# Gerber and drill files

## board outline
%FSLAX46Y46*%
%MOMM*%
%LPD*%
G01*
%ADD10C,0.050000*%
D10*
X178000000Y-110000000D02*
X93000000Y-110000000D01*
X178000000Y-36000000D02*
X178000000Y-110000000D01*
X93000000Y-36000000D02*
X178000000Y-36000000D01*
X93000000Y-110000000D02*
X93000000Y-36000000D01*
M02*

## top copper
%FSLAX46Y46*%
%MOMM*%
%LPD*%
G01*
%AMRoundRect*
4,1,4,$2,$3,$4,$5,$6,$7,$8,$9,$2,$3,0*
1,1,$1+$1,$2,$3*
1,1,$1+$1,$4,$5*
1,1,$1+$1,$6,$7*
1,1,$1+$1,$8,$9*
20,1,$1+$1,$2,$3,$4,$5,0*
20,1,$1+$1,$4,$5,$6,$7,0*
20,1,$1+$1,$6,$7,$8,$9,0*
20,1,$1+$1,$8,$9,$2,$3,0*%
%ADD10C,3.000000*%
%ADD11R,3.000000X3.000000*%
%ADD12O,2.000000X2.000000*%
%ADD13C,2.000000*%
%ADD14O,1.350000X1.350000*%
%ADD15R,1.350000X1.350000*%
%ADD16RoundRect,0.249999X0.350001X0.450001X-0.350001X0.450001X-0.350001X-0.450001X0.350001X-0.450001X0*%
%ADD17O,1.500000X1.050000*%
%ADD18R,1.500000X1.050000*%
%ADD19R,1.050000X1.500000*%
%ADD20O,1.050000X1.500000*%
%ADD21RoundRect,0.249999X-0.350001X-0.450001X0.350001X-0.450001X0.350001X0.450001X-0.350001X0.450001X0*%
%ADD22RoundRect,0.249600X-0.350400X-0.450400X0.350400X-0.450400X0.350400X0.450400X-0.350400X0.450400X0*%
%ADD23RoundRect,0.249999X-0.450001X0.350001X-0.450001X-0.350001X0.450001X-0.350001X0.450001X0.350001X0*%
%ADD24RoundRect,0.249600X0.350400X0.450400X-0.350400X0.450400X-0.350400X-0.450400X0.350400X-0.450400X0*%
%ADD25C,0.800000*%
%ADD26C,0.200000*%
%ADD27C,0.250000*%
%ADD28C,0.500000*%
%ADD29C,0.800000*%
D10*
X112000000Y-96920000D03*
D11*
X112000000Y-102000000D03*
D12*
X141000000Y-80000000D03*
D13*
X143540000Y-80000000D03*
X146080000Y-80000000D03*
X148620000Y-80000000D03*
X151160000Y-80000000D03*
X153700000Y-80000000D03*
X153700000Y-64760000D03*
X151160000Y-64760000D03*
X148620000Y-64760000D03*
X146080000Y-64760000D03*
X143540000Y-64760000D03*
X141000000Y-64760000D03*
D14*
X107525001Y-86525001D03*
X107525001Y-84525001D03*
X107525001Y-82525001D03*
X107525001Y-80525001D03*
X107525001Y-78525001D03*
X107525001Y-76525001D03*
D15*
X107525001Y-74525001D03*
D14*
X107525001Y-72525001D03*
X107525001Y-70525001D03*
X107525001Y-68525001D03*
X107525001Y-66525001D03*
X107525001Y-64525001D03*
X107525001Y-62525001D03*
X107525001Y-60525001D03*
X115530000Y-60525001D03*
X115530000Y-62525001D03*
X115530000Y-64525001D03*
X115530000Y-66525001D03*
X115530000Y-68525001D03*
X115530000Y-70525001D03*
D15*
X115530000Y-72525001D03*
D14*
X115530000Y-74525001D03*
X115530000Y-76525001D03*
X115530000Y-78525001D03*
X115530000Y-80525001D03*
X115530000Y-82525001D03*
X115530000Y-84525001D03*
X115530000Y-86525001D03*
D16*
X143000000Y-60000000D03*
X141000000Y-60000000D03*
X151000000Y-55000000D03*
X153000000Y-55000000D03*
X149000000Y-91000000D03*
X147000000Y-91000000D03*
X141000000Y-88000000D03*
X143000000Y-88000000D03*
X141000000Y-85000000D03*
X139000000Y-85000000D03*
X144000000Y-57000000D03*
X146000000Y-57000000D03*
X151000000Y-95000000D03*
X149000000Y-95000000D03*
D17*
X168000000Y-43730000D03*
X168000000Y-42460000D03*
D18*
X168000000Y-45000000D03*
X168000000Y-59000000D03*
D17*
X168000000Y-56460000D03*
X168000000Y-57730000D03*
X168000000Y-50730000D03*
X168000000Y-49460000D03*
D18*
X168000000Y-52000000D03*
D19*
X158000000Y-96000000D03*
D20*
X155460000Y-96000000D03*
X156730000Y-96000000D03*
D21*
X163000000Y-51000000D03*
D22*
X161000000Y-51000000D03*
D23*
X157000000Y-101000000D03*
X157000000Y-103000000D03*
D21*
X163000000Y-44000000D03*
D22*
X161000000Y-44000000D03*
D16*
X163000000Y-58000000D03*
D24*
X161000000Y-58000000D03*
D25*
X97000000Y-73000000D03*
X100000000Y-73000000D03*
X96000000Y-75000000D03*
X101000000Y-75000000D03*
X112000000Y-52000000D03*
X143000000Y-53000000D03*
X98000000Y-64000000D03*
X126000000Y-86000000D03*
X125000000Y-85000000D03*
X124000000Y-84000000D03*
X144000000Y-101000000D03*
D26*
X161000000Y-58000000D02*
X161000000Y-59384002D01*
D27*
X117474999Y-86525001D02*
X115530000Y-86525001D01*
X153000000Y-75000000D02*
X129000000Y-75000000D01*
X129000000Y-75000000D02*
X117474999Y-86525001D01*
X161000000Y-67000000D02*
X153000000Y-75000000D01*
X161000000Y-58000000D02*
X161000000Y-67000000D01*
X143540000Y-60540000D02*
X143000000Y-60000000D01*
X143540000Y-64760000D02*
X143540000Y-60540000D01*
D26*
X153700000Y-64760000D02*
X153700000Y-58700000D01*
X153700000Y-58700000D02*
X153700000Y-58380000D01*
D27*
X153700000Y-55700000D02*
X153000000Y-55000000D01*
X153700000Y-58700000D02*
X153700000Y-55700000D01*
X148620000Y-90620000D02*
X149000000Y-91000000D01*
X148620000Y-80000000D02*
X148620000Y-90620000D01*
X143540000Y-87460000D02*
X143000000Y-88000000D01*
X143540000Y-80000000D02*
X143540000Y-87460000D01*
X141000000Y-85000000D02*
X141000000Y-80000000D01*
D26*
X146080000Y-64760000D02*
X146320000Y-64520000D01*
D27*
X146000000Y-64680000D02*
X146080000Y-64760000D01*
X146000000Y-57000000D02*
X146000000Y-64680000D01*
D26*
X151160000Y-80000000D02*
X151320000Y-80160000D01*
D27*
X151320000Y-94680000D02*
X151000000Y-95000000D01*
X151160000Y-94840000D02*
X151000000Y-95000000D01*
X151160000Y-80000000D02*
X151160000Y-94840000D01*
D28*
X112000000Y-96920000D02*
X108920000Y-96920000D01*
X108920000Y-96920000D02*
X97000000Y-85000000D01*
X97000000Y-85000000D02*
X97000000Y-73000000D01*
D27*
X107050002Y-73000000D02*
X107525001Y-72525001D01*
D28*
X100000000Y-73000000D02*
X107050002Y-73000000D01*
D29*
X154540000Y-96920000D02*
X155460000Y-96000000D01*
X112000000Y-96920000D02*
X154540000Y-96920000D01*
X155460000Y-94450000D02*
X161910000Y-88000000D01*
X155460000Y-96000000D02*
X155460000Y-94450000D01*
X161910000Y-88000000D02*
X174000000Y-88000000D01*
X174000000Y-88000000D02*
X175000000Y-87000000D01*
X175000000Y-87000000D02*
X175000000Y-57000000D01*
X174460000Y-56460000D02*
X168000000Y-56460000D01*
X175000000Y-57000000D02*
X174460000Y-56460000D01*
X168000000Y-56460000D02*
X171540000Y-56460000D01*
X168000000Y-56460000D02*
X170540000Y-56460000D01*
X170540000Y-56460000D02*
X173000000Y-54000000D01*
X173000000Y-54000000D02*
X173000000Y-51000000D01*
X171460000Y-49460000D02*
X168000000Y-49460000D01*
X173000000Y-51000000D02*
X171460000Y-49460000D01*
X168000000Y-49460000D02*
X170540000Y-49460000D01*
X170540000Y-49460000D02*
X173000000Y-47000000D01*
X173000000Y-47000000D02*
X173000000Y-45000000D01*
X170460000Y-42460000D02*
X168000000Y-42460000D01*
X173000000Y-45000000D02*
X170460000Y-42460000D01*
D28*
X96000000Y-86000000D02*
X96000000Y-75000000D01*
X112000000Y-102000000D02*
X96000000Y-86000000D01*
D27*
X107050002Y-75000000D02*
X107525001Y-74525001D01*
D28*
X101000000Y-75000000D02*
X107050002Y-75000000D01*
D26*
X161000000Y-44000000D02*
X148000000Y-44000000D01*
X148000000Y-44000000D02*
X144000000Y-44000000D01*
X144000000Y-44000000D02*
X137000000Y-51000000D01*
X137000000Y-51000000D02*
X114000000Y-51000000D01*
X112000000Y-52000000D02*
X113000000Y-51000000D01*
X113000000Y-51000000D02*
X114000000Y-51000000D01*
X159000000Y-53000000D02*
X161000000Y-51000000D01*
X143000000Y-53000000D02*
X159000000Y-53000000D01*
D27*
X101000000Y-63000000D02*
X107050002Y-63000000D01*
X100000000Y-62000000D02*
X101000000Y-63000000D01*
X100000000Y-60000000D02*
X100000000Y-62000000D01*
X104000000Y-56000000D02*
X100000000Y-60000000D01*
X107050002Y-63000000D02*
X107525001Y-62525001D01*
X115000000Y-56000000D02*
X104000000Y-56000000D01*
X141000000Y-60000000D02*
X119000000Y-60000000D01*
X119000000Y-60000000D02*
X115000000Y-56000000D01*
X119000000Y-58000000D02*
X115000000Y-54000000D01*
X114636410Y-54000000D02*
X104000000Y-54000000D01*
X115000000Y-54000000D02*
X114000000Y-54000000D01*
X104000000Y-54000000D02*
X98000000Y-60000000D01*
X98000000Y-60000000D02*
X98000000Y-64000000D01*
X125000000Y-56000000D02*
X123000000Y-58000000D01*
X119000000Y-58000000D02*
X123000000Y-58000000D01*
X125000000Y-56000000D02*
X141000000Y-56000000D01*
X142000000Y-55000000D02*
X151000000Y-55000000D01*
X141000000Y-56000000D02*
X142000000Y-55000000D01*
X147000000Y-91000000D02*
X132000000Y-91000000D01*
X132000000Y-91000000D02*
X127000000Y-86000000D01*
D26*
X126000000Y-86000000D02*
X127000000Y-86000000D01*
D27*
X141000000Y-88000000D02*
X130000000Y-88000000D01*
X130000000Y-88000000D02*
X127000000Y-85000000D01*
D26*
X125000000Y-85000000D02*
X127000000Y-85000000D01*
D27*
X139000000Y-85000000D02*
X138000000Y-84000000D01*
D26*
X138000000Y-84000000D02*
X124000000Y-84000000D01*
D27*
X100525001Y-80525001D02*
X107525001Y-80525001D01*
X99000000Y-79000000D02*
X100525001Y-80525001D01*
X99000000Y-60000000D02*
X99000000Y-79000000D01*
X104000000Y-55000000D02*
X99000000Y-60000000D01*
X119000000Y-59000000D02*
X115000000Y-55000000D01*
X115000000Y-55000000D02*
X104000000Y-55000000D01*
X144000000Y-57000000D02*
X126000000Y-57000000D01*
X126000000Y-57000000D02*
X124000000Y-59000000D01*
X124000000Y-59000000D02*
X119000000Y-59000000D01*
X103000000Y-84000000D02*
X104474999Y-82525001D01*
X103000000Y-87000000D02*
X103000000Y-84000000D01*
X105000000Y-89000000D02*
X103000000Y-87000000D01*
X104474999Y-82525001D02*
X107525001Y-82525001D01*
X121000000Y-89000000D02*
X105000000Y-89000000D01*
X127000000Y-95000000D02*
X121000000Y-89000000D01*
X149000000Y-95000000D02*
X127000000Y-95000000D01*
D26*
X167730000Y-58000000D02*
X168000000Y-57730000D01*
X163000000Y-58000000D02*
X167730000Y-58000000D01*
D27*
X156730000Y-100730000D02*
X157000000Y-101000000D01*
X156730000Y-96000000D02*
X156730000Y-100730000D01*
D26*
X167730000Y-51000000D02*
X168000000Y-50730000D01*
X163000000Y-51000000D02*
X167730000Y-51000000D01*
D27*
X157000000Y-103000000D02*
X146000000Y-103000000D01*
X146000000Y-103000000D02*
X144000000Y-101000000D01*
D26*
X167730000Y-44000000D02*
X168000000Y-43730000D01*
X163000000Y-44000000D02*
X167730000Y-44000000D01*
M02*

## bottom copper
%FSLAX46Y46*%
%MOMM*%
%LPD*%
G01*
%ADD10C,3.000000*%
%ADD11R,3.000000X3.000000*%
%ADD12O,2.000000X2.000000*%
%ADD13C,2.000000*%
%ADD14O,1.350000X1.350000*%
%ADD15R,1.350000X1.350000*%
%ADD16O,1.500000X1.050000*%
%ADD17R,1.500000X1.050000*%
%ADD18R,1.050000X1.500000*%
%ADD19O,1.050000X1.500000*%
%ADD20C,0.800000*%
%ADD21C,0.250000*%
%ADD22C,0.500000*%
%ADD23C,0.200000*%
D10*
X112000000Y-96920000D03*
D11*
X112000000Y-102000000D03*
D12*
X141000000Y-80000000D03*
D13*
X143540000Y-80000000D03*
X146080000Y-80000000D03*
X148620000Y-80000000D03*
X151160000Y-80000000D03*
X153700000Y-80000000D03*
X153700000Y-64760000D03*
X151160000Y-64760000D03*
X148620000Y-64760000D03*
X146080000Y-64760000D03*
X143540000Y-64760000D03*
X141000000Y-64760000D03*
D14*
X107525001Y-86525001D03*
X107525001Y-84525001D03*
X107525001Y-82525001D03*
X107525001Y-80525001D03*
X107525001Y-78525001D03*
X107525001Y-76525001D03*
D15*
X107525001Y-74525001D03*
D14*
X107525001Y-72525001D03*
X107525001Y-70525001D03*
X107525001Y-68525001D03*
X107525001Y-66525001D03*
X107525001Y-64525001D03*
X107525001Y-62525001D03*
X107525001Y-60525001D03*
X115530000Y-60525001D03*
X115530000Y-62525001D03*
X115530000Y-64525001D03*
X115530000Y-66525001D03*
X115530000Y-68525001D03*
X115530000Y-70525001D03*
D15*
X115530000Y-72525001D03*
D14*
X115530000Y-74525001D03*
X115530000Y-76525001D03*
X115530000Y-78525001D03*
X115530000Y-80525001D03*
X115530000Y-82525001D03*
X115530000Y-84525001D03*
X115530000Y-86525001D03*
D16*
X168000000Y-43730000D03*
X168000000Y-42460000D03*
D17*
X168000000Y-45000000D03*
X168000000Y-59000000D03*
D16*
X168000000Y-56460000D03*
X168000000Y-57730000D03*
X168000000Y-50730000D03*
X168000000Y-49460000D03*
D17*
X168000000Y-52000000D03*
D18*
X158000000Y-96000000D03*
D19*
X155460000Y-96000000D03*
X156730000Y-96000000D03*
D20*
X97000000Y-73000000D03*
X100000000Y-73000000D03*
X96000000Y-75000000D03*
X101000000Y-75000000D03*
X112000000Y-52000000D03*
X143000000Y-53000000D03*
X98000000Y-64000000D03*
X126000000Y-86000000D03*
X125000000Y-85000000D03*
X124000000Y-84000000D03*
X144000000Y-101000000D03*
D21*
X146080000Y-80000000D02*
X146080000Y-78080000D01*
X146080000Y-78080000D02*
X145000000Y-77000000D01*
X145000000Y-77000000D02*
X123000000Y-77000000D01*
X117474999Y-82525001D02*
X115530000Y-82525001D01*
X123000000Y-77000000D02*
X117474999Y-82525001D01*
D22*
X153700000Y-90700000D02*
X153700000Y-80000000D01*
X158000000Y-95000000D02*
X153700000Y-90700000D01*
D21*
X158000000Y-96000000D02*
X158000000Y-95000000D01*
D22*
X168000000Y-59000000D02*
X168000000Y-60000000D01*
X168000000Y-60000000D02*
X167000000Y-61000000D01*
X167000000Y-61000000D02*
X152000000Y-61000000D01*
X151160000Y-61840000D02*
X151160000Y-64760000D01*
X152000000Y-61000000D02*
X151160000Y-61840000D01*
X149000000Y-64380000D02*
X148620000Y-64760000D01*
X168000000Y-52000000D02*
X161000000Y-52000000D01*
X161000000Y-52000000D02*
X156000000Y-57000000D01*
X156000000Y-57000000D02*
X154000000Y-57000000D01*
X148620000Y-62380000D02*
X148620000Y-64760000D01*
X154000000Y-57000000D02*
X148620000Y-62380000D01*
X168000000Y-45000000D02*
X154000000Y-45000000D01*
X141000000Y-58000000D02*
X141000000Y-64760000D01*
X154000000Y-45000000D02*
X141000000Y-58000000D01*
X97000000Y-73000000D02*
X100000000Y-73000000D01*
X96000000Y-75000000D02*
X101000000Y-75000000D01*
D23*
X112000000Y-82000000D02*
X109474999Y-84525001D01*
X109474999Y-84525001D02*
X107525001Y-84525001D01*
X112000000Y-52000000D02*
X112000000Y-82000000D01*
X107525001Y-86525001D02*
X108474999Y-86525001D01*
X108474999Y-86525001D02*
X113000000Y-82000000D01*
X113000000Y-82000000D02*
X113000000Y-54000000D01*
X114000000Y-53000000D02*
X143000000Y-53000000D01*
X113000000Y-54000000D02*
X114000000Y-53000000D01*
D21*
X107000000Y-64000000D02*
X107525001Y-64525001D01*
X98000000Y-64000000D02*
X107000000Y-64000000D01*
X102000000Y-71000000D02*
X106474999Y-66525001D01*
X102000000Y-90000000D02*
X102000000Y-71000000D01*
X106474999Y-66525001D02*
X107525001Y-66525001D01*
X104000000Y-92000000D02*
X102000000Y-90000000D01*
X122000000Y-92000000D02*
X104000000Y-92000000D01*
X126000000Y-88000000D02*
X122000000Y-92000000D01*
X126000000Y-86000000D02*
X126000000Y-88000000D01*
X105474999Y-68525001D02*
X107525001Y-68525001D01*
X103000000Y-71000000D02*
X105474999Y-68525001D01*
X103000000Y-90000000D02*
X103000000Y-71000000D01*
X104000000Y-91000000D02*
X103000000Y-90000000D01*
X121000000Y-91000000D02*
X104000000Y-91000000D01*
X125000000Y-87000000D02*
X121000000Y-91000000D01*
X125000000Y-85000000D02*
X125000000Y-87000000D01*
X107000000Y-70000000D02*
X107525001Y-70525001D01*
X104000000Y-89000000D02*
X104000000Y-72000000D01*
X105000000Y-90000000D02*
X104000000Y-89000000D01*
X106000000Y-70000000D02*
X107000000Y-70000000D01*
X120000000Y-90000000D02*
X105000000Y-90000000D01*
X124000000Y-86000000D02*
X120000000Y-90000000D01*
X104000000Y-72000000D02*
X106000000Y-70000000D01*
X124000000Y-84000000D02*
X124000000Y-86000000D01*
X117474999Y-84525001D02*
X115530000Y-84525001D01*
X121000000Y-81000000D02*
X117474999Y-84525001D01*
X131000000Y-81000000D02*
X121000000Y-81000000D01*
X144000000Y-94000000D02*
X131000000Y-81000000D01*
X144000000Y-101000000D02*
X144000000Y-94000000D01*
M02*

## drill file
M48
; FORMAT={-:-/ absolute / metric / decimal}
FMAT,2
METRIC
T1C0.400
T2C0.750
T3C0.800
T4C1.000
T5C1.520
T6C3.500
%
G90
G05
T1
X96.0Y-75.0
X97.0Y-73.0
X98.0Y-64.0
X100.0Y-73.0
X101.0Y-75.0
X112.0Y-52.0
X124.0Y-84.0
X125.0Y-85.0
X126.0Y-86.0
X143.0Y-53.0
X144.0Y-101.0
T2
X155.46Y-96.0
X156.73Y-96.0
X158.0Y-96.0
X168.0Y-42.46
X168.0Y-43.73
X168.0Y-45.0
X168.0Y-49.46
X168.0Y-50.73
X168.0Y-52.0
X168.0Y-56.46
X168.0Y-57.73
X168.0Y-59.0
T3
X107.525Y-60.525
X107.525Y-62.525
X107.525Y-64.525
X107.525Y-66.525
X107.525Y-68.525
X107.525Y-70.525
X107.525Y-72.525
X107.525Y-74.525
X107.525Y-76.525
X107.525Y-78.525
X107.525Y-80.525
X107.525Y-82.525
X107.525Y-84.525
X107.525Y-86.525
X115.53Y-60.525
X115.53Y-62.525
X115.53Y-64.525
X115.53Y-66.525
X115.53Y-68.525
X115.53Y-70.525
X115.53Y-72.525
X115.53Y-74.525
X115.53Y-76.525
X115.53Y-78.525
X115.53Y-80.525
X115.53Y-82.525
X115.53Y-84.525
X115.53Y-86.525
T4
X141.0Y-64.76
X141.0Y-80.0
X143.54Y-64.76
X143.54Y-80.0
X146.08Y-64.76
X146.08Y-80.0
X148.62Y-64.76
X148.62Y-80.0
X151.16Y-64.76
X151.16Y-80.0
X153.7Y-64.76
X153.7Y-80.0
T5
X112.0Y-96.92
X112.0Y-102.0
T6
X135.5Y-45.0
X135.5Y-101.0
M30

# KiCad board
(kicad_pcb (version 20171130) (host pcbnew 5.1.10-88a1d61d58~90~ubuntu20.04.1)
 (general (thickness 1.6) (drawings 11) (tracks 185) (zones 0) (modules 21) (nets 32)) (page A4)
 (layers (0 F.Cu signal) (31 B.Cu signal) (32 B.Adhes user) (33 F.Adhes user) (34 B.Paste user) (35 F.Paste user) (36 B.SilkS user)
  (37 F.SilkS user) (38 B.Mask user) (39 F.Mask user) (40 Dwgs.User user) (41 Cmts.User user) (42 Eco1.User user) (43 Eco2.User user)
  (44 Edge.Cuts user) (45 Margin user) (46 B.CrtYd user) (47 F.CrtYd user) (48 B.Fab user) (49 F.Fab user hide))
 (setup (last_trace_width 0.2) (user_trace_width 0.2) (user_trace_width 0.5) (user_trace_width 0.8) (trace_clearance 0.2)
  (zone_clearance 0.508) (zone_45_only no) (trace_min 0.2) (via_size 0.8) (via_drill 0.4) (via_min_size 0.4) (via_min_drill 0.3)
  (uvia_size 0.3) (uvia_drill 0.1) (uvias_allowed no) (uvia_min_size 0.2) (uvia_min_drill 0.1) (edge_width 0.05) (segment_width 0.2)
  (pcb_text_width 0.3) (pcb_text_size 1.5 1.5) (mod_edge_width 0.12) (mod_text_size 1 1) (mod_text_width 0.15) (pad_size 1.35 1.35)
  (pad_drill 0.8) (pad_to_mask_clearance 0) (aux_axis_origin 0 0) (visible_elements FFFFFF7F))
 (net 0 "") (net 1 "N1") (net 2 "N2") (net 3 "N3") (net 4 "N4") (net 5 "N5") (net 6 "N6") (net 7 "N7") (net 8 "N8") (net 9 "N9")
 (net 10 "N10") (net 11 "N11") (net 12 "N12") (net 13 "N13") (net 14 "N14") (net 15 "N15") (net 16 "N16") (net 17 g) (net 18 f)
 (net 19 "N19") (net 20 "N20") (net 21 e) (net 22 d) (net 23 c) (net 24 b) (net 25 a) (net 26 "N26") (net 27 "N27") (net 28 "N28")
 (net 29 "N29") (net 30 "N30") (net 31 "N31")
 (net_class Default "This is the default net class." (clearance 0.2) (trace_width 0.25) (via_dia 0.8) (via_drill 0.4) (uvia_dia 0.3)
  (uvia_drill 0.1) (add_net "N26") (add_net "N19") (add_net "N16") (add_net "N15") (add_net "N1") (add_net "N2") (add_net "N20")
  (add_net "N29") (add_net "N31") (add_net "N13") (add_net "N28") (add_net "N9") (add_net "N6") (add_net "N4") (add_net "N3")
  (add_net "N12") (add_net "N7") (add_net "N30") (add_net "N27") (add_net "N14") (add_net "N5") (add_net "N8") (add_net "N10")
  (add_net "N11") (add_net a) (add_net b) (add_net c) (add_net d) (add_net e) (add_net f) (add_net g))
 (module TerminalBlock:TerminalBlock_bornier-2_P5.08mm (layer F.Cu) (at 112 102 90)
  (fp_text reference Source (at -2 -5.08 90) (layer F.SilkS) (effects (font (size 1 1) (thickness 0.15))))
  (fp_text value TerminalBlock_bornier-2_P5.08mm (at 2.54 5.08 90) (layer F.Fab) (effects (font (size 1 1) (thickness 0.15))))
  (pad 2 thru_hole circle (at 5.08 0 90) (size 3 3) (drill 1.52) (layers *.Cu *.Mask) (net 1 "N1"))
  (pad 1 thru_hole rect (at 0 0 90) (size 3 3) (drill 1.52) (layers *.Cu *.Mask) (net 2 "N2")))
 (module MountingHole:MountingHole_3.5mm (layer F.Cu) (at 135.5 45)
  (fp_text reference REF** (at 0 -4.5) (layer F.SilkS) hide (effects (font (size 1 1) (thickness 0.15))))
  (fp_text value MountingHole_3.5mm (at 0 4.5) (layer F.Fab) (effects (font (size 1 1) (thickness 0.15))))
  (pad 1 np_thru_hole circle (at 0 0) (size 3.5 3.5) (drill 3.5) (layers *.Cu *.Mask)))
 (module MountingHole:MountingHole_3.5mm (layer F.Cu) (at 135.5 101)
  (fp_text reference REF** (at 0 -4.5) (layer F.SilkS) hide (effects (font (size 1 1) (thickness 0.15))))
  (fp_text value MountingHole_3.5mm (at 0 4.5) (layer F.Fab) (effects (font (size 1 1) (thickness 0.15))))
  (pad 1 np_thru_hole circle (at 0 0) (size 3.5 3.5) (drill 3.5) (layers *.Cu *.Mask)))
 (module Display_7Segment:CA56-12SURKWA (layer F.Cu) (at 141 80 90)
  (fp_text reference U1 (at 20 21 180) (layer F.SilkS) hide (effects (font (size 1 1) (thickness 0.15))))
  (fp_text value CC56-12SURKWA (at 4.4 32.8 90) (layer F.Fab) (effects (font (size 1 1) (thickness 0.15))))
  (pad 1 thru_hole oval (at 0 0 90) (size 2 2) (drill 1) (layers *.Cu *.Mask) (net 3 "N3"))
  (pad 2 thru_hole circle (at 0 2.54 90) (size 2 2) (drill 1) (layers *.Cu *.Mask) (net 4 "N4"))
  (pad 3 thru_hole circle (at 0 5.08 90) (size 2 2) (drill 1) (layers *.Cu *.Mask) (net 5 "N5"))
  (pad 4 thru_hole circle (at 0 7.62 90) (size 2 2) (drill 1) (layers *.Cu *.Mask) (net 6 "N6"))
  (pad 5 thru_hole circle (at 0 10.16 90) (size 2 2) (drill 1) (layers *.Cu *.Mask) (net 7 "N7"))
  (pad 6 thru_hole circle (at 0 12.7 90) (size 2 2) (drill 1) (layers *.Cu *.Mask) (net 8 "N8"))
  (pad 7 thru_hole circle (at 15.24 12.7 90) (size 2 2) (drill 1) (layers *.Cu *.Mask) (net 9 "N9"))
  (pad 8 thru_hole circle (at 15.24 10.16 90) (size 2 2) (drill 1) (layers *.Cu *.Mask) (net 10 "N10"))
  (pad 9 thru_hole circle (at 15.24 7.62 90) (size 2 2) (drill 1) (layers *.Cu *.Mask) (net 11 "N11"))
  (pad 10 thru_hole circle (at 15.24 5.08 90) (size 2 2) (drill 1) (layers *.Cu *.Mask) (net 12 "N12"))
  (pad 11 thru_hole circle (at 15.24 2.54 90) (size 2 2) (drill 1) (layers *.Cu *.Mask) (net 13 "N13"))
  (pad 12 thru_hole circle (at 15.24 0 90) (size 2 2) (drill 1) (layers *.Cu *.Mask) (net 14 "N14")))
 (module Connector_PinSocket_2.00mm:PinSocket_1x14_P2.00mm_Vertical (layer F.Cu) (at 107.525001 60.525001)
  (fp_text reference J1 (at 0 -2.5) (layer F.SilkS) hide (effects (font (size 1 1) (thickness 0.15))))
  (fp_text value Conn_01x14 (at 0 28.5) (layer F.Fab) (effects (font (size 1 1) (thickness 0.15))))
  (pad 14 thru_hole oval (at 0 26) (size 1.35 1.35) (drill 0.8) (layers *.Cu *.Mask) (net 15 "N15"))
  (pad 13 thru_hole oval (at 0 24) (size 1.35 1.35) (drill 0.8) (layers *.Cu *.Mask) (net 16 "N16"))
  (pad 12 thru_hole oval (at 0 22) (size 1.35 1.35) (drill 0.8) (layers *.Cu *.Mask) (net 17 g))
  (pad 11 thru_hole oval (at 0 20) (size 1.35 1.35) (drill 0.8) (layers *.Cu *.Mask) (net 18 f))
  (pad 10 thru_hole oval (at 0 18) (size 1.35 1.35) (drill 0.8) (layers *.Cu *.Mask) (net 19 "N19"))
  (pad 9 thru_hole oval (at 0 16) (size 1.35 1.35) (drill 0.8) (layers *.Cu *.Mask) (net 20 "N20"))
  (pad 8 thru_hole rect (at 0 14) (size 1.35 1.35) (drill 0.8) (layers *.Cu *.Mask) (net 2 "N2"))
  (pad 7 thru_hole oval (at 0 12) (size 1.35 1.35) (drill 0.8) (layers *.Cu *.Mask) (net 1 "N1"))
  (pad 6 thru_hole oval (at 0 10) (size 1.35 1.35) (drill 0.8) (layers *.Cu *.Mask) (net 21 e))
  (pad 5 thru_hole oval (at 0 8) (size 1.35 1.35) (drill 0.8) (layers *.Cu *.Mask) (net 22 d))
  (pad 4 thru_hole oval (at 0 6) (size 1.35 1.35) (drill 0.8) (layers *.Cu *.Mask) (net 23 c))
  (pad 3 thru_hole oval (at 0 4) (size 1.35 1.35) (drill 0.8) (layers *.Cu *.Mask) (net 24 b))
  (pad 2 thru_hole oval (at 0 2) (size 1.35 1.35) (drill 0.8) (layers *.Cu *.Mask) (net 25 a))
  (pad 1 thru_hole oval (at 0 0) (size 1.35 1.35) (drill 0.8) (layers *.Cu *.Mask) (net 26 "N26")))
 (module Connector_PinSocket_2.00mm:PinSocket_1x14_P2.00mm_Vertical (layer F.Cu) (at 115.53 60.525001)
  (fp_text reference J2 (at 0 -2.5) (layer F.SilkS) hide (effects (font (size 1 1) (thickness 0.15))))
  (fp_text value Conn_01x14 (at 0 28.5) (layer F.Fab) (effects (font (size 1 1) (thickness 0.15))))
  (pad 28 thru_hole oval (at 0 0) (size 1.35 1.35) (drill 0.8) (layers *.Cu *.Mask))
  (pad 27 thru_hole oval (at 0 2) (size 1.35 1.35) (drill 0.8) (layers *.Cu *.Mask))
  (pad 26 thru_hole oval (at 0 4) (size 1.35 1.35) (drill 0.8) (layers *.Cu *.Mask))
  (pad 25 thru_hole oval (at 0 6) (size 1.35 1.35) (drill 0.8) (layers *.Cu *.Mask))
  (pad 24 thru_hole oval (at 0 8) (size 1.35 1.35) (drill 0.8) (layers *.Cu *.Mask))
  (pad 23 thru_hole oval (at 0 10) (size 1.35 1.35) (drill 0.8) (layers *.Cu *.Mask))
  (pad 22 thru_hole rect (at 0 12) (size 1.35 1.35) (drill 0.8) (layers *.Cu *.Mask))
  (pad 21 thru_hole oval (at 0 14) (size 1.35 1.35) (drill 0.8) (layers *.Cu *.Mask))
  (pad 20 thru_hole oval (at 0 16) (size 1.35 1.35) (drill 0.8) (layers *.Cu *.Mask))
  (pad 19 thru_hole oval (at 0 18) (size 1.35 1.35) (drill 0.8) (layers *.Cu *.Mask))
  (pad 18 thru_hole oval (at 0 20) (size 1.35 1.35) (drill 0.8) (layers *.Cu *.Mask))
  (pad 17 thru_hole oval (at 0 22) (size 1.35 1.35) (drill 0.8) (layers *.Cu *.Mask) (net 5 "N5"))
  (pad 16 thru_hole oval (at 0 24) (size 1.35 1.35) (drill 0.8) (layers *.Cu *.Mask) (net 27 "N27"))
  (pad 15 thru_hole oval (at 0 26) (size 1.35 1.35) (drill 0.8) (layers *.Cu *.Mask)))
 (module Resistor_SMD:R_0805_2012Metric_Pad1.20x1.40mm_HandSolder (layer F.Cu) (at 142 60 180)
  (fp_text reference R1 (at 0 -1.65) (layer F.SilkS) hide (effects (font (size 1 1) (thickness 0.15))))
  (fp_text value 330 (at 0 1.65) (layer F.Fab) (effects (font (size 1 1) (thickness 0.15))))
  (pad 1 smd roundrect (at -1 0 180) (size 1.2 1.4) (layers F.Cu F.Paste F.Mask) (roundrect_rratio 0.2083325) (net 13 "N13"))
  (pad 2 smd roundrect (at 1 0 180) (size 1.2 1.4) (layers F.Cu F.Paste F.Mask) (roundrect_rratio 0.2083325) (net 25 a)))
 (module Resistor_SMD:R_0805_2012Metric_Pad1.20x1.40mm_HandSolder (layer F.Cu) (at 152 55 180)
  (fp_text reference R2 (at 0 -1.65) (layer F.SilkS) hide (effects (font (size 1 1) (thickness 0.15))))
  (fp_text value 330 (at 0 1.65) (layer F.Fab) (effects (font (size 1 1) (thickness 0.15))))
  (pad 2 smd roundrect (at 1 0 180) (size 1.2 1.4) (layers F.Cu F.Paste F.Mask) (roundrect_rratio 0.2083325) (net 24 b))
  (pad 1 smd roundrect (at -1 0 180) (size 1.2 1.4) (layers F.Cu F.Paste F.Mask) (roundrect_rratio 0.2083325) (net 9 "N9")))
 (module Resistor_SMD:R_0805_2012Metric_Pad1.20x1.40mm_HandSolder (layer F.Cu) (at 148 91 180)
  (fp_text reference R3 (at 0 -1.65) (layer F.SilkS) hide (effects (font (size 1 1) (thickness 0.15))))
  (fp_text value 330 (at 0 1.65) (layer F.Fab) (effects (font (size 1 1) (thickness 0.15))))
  (pad 1 smd roundrect (at -1 0 180) (size 1.2 1.4) (layers F.Cu F.Paste F.Mask) (roundrect_rratio 0.2083325) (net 6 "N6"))
  (pad 2 smd roundrect (at 1 0 180) (size 1.2 1.4) (layers F.Cu F.Paste F.Mask) (roundrect_rratio 0.2083325) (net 23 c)))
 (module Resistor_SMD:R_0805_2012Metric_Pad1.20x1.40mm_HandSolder (layer F.Cu) (at 142 88 180)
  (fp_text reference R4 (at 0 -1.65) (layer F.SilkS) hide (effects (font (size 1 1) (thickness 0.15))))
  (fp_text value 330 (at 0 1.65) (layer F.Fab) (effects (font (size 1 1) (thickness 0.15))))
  (pad 2 smd roundrect (at 1 0 180) (size 1.2 1.4) (layers F.Cu F.Paste F.Mask) (roundrect_rratio 0.2083325) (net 22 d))
  (pad 1 smd roundrect (at -1 0 180) (size 1.2 1.4) (layers F.Cu F.Paste F.Mask) (roundrect_rratio 0.2083325) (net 4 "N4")))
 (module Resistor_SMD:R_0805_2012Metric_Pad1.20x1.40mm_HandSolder (layer F.Cu) (at 140 85 180)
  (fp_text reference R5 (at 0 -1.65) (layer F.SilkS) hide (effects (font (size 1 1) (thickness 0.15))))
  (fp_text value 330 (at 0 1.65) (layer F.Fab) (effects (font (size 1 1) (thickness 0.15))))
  (pad 1 smd roundrect (at -1 0 180) (size 1.2 1.4) (layers F.Cu F.Paste F.Mask) (roundrect_rratio 0.2083325) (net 3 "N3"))
  (pad 2 smd roundrect (at 1 0 180) (size 1.2 1.4) (layers F.Cu F.Paste F.Mask) (roundrect_rratio 0.2083325) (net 21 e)))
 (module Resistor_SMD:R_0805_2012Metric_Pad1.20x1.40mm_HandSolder (layer F.Cu) (at 145 57 180)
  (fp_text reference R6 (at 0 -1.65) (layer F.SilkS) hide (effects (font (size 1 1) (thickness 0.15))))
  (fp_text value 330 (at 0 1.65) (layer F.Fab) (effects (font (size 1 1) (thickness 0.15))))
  (pad 2 smd roundrect (at 1 0 180) (size 1.2 1.4) (layers F.Cu F.Paste F.Mask) (roundrect_rratio 0.2083325) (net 18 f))
  (pad 1 smd roundrect (at -1 0 180) (size 1.2 1.4) (layers F.Cu F.Paste F.Mask) (roundrect_rratio 0.2083325) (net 12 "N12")))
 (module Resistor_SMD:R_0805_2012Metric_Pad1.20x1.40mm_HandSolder (layer F.Cu) (at 150 95 180)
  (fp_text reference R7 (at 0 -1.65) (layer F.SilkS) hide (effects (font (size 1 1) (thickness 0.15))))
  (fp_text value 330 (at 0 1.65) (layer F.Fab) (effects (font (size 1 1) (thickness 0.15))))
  (pad 1 smd roundrect (at -1 0 180) (size 1.2 1.4) (layers F.Cu F.Paste F.Mask) (roundrect_rratio 0.2083325) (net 7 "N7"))
  (pad 2 smd roundrect (at 1 0 180) (size 1.2 1.4) (layers F.Cu F.Paste F.Mask) (roundrect_rratio 0.2083325) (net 17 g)))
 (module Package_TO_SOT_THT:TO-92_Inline (layer F.Cu) (at 168 45 90)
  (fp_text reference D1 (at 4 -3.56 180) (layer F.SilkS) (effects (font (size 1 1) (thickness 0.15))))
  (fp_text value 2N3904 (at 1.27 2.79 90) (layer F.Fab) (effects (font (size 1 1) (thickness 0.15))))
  (pad 2 thru_hole oval (at 1.27 0 90) (size 1.05 1.5) (drill 0.75) (layers *.Cu *.Mask) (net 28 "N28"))
  (pad 3 thru_hole oval (at 2.54 0 90) (size 1.05 1.5) (drill 0.75) (layers *.Cu *.Mask) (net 1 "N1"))
  (pad 1 thru_hole rect (at 0 0 90) (size 1.05 1.5) (drill 0.75) (layers *.Cu *.Mask) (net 14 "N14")))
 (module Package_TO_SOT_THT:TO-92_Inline (layer F.Cu) (at 168 59 90)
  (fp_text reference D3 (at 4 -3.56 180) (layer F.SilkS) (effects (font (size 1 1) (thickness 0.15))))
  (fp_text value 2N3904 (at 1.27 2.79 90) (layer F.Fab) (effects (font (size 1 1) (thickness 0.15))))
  (pad 1 thru_hole rect (at 0 0 90) (size 1.05 1.5) (drill 0.75) (layers *.Cu *.Mask) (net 10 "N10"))
  (pad 3 thru_hole oval (at 2.54 0 90) (size 1.05 1.5) (drill 0.75) (layers *.Cu *.Mask) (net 1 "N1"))
  (pad 2 thru_hole oval (at 1.27 0 90) (size 1.05 1.5) (drill 0.75) (layers *.Cu *.Mask) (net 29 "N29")))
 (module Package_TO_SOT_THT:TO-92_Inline (layer F.Cu) (at 168 52 90)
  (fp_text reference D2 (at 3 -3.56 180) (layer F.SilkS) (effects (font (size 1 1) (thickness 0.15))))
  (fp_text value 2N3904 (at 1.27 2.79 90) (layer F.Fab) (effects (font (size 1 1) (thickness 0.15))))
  (pad 2 thru_hole oval (at 1.27 0 90) (size 1.05 1.5) (drill 0.75) (layers *.Cu *.Mask) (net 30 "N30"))
  (pad 3 thru_hole oval (at 2.54 0 90) (size 1.05 1.5) (drill 0.75) (layers *.Cu *.Mask) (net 1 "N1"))
  (pad 1 thru_hole rect (at 0 0 90) (size 1.05 1.5) (drill 0.75) (layers *.Cu *.Mask) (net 11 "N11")))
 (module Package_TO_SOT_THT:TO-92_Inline (layer F.Cu) (at 158 96 180)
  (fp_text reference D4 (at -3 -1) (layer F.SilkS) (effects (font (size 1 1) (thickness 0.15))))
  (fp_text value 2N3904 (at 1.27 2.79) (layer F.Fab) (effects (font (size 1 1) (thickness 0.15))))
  (pad 1 thru_hole rect (at 0 0 180) (size 1.05 1.5) (drill 0.75) (layers *.Cu *.Mask) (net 8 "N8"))
  (pad 3 thru_hole oval (at 2.54 0 180) (size 1.05 1.5) (drill 0.75) (layers *.Cu *.Mask) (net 1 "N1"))
  (pad 2 thru_hole oval (at 1.27 0 180) (size 1.05 1.5) (drill 0.75) (layers *.Cu *.Mask) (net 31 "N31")))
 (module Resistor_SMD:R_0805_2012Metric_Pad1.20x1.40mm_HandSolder (layer F.Cu) (at 162 51)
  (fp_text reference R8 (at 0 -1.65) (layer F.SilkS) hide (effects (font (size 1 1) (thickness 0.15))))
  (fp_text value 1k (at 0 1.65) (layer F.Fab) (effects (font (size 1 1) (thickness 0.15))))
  (pad 2 smd roundrect (at 1 0) (size 1.2 1.4) (layers F.Cu F.Paste F.Mask) (roundrect_rratio 0.2083325) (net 30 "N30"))
  (pad 1 smd roundrect (at -1 0) (size 1.2 1.4) (layers F.Cu F.Paste F.Mask) (roundrect_rratio 0.208) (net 15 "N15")))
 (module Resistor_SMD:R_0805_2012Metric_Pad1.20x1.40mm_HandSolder (layer F.Cu) (at 157 102 270)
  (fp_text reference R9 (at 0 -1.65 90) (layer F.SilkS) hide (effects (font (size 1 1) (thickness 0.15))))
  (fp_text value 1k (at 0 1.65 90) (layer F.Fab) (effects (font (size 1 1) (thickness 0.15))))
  (pad 1 smd roundrect (at -1 0 270) (size 1.2 1.4) (layers F.Cu F.Paste F.Mask) (roundrect_rratio 0.2083325) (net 31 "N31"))
  (pad 2 smd roundrect (at 1 0 270) (size 1.2 1.4) (layers F.Cu F.Paste F.Mask) (roundrect_rratio 0.2083325) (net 27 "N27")))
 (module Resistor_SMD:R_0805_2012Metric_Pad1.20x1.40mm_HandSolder (layer F.Cu) (at 162 44)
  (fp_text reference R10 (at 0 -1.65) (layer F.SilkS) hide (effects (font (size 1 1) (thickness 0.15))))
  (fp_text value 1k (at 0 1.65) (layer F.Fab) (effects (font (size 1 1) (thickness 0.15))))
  (pad 2 smd roundrect (at 1 0) (size 1.2 1.4) (layers F.Cu F.Paste F.Mask) (roundrect_rratio 0.2083325) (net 28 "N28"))
  (pad 1 smd roundrect (at -1 0) (size 1.2 1.4) (layers F.Cu F.Paste F.Mask) (roundrect_rratio 0.208) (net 16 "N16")))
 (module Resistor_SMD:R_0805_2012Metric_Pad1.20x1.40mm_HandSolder (layer F.Cu) (at 162 58 180)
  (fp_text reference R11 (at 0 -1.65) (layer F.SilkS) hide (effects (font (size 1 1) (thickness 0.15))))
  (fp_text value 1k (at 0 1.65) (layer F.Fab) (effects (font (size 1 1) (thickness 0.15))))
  (pad 1 smd roundrect (at -1 0 180) (size 1.2 1.4) (layers F.Cu F.Paste F.Mask) (roundrect_rratio 0.2083325) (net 29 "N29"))
  (pad 2 smd roundrect (at 1 0 180) (size 1.2 1.4) (layers F.Cu F.Paste F.Mask) (roundrect_rratio 0.208)))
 (gr_line (start 178 110) (end 93 110) (layer Edge.Cuts) (width 0.05))
 (gr_line (start 178 36) (end 178 110) (layer Edge.Cuts) (width 0.05))
 (gr_line (start 93 36) (end 178 36) (layer Edge.Cuts) (width 0.05))
 (gr_line (start 93 110) (end 93 36) (layer Edge.Cuts) (width 0.05))
 (segment (start 161 58) (end 161 59.384002) (width 0.2) (layer F.Cu) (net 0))
 (segment (start 117.474999 86.525001) (end 115.53 86.525001) (width 0.25) (layer F.Cu) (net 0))
 (segment (start 153 75) (end 129 75) (width 0.25) (layer F.Cu) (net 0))
 (segment (start 129 75) (end 117.474999 86.525001) (width 0.25) (layer F.Cu) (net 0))
 (segment (start 161 67) (end 153 75) (width 0.25) (layer F.Cu) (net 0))
 (segment (start 161 58) (end 161 67) (width 0.25) (layer F.Cu) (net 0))
 (segment (start 146.08 80) (end 146.08 78.08) (width 0.25) (layer B.Cu) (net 5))
 (segment (start 146.08 78.08) (end 145 77) (width 0.25) (layer B.Cu) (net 5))
 (segment (start 145 77) (end 123 77) (width 0.25) (layer B.Cu) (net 5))
 (segment (start 117.474999 82.525001) (end 115.53 82.525001) (width 0.25) (layer B.Cu) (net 5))
 (segment (start 123 77) (end 117.474999 82.525001) (width 0.25) (layer B.Cu) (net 5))
 (segment (start 153.7 90.7) (end 153.7 80) (width 0.5) (layer B.Cu) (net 8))
 (segment (start 158 95) (end 153.7 90.7) (width 0.5) (layer B.Cu) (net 8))
 (segment (start 158 96) (end 158 95) (width 0.25) (layer B.Cu) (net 8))
 (segment (start 168 59) (end 168 60) (width 0.5) (layer B.Cu) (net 10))
 (segment (start 168 60) (end 167 61) (width 0.5) (layer B.Cu) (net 10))
 (segment (start 167 61) (end 152 61) (width 0.5) (layer B.Cu) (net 10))
 (segment (start 151.16 61.84) (end 151.16 64.76) (width 0.5) (layer B.Cu) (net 10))
 (segment (start 152 61) (end 151.16 61.84) (width 0.5) (layer B.Cu) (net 10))
 (segment (start 149 64.38) (end 148.62 64.76) (width 0.5) (layer B.Cu) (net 11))
 (segment (start 168 52) (end 161 52) (width 0.5) (layer B.Cu) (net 11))
 (segment (start 161 52) (end 156 57) (width 0.5) (layer B.Cu) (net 11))
 (segment (start 156 57) (end 154 57) (width 0.5) (layer B.Cu) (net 11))
 (segment (start 148.62 62.38) (end 148.62 64.76) (width 0.5) (layer B.Cu) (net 11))
 (segment (start 154 57) (end 148.62 62.38) (width 0.5) (layer B.Cu) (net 11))
 (segment (start 168 45) (end 154 45) (width 0.5) (layer B.Cu) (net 14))
 (segment (start 141 58) (end 141 64.76) (width 0.5) (layer B.Cu) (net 14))
 (segment (start 154 45) (end 141 58) (width 0.5) (layer B.Cu) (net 14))
 (segment (start 143.54 60.54) (end 143 60) (width 0.25) (layer F.Cu) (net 13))
 (segment (start 143.54 64.76) (end 143.54 60.54) (width 0.25) (layer F.Cu) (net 13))
 (segment (start 153.7 64.76) (end 153.7 58.7) (width 0.2) (layer F.Cu) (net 9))
 (segment (start 153.7 58.7) (end 153.7 58.38) (width 0.2) (layer F.Cu) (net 9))
 (segment (start 153.7 55.7) (end 153 55) (width 0.25) (layer F.Cu) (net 9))
 (segment (start 153.7 58.7) (end 153.7 55.7) (width 0.25) (layer F.Cu) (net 9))
 (segment (start 148.62 90.62) (end 149 91) (width 0.25) (layer F.Cu) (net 6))
 (segment (start 148.62 80) (end 148.62 90.62) (width 0.25) (layer F.Cu) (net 6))
 (segment (start 143.54 87.46) (end 143 88) (width 0.25) (layer F.Cu) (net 4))
 (segment (start 143.54 80) (end 143.54 87.46) (width 0.25) (layer F.Cu) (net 4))
 (segment (start 141 85) (end 141 80) (width 0.25) (layer F.Cu) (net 3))
 (segment (start 146.08 64.76) (end 146.32 64.52) (width 0.2) (layer F.Cu) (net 12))
 (segment (start 146 64.68) (end 146.08 64.76) (width 0.25) (layer F.Cu) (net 12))
 (segment (start 146 57) (end 146 64.68) (width 0.25) (layer F.Cu) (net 12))
 (segment (start 151.16 80) (end 151.32 80.16) (width 0.2) (layer F.Cu) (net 7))
 (segment (start 151.32 94.68) (end 151 95) (width 0.25) (layer F.Cu) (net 7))
 (segment (start 151.16 94.84) (end 151 95) (width 0.25) (layer F.Cu) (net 7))
 (segment (start 151.16 80) (end 151.16 94.84) (width 0.25) (layer F.Cu) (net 7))
 (segment (start 112 96.92) (end 108.92 96.92) (width 0.5) (layer F.Cu) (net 1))
 (segment (start 108.92 96.92) (end 97 85) (width 0.5) (layer F.Cu) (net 1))
 (via (at 97 73) (size 0.8) (drill 0.4) (layers F.Cu B.Cu) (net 1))
 (segment (start 97 85) (end 97 73) (width 0.5) (layer F.Cu) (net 1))
 (via (at 100 73) (size 0.8) (drill 0.4) (layers F.Cu B.Cu) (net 1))
 (segment (start 97 73) (end 100 73) (width 0.5) (layer B.Cu) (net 1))
 (segment (start 107.050002 73) (end 107.525001 72.525001) (width 0.25) (layer F.Cu) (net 1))
 (segment (start 100 73) (end 107.050002 73) (width 0.5) (layer F.Cu) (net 1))
 (segment (start 154.54 96.92) (end 155.46 96) (width 0.8) (layer F.Cu) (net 1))
 (segment (start 112 96.92) (end 154.54 96.92) (width 0.8) (layer F.Cu) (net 1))
 (segment (start 155.46 94.45) (end 161.91 88) (width 0.8) (layer F.Cu) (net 1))
 (segment (start 155.46 96) (end 155.46 94.45) (width 0.8) (layer F.Cu) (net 1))
 (segment (start 161.91 88) (end 174 88) (width 0.8) (layer F.Cu) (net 1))
 (segment (start 174 88) (end 175 87) (width 0.8) (layer F.Cu) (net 1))
 (segment (start 175 87) (end 175 57) (width 0.8) (layer F.Cu) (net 1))
 (segment (start 174.46 56.46) (end 168 56.46) (width 0.8) (layer F.Cu) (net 1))
 (segment (start 175 57) (end 174.46 56.46) (width 0.8) (layer F.Cu) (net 1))
 (segment (start 168 56.46) (end 171.54 56.46) (width 0.8) (layer F.Cu) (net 1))
 (segment (start 168 56.46) (end 170.54 56.46) (width 0.8) (layer F.Cu) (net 1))
 (segment (start 170.54 56.46) (end 173 54) (width 0.8) (layer F.Cu) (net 1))
 (segment (start 173 54) (end 173 51) (width 0.8) (layer F.Cu) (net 1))
 (segment (start 171.46 49.46) (end 168 49.46) (width 0.8) (layer F.Cu) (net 1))
 (segment (start 173 51) (end 171.46 49.46) (width 0.8) (layer F.Cu) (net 1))
 (segment (start 168 49.46) (end 170.54 49.46) (width 0.8) (layer F.Cu) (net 1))
 (segment (start 170.54 49.46) (end 173 47) (width 0.8) (layer F.Cu) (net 1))
 (segment (start 173 47) (end 173 45) (width 0.8) (layer F.Cu) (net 1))
 (segment (start 170.46 42.46) (end 168 42.46) (width 0.8) (layer F.Cu) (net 1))
 (segment (start 173 45) (end 170.46 42.46) (width 0.8) (layer F.Cu) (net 1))
 (via (at 96 75) (size 0.8) (drill 0.4) (layers F.Cu B.Cu) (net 2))
 (segment (start 96 86) (end 96 75) (width 0.5) (layer F.Cu) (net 2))
 (segment (start 112 102) (end 96 86) (width 0.5) (layer F.Cu) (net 2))
 (via (at 101 75) (size 0.8) (drill 0.4) (layers F.Cu B.Cu) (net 2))
 (segment (start 96 75) (end 101 75) (width 0.5) (layer B.Cu) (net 2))
 (segment (start 107.050002 75) (end 107.525001 74.525001) (width 0.25) (layer F.Cu) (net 2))
 (segment (start 101 75) (end 107.050002 75) (width 0.5) (layer F.Cu) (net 2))
 (segment (start 161 44) (end 148 44) (width 0.2) (layer F.Cu) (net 16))
 (segment (start 148 44) (end 144 44) (width 0.2) (layer F.Cu) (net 16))
 (segment (start 144 44) (end 137 51) (width 0.2) (layer F.Cu) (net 16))
 (via (at 112 52) (size 0.8) (drill 0.4) (layers F.Cu B.Cu) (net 16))
 (segment (start 137 51) (end 114 51) (width 0.2) (layer F.Cu) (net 16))
 (segment (start 112 52) (end 113 51) (width 0.2) (layer F.Cu) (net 16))
 (segment (start 112 82) (end 109.474999 84.525001) (width 0.2) (layer B.Cu) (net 16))
 (segment (start 109.474999 84.525001) (end 107.525001 84.525001) (width 0.2) (layer B.Cu) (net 16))
 (segment (start 112 52) (end 112 82) (width 0.2) (layer B.Cu) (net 16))
 (segment (start 113 51) (end 114 51) (width 0.2) (layer F.Cu) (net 16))
 (segment (start 107.525001 86.525001) (end 108.474999 86.525001) (width 0.2) (layer B.Cu) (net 15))
 (segment (start 108.474999 86.525001) (end 113 82) (width 0.2) (layer B.Cu) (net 15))
 (segment (start 113 82) (end 113 54) (width 0.2) (layer B.Cu) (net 15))
 (via (at 143 53) (size 0.8) (drill 0.4) (layers F.Cu B.Cu) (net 15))
 (segment (start 114 53) (end 143 53) (width 0.2) (layer B.Cu) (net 15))
 (segment (start 113 54) (end 114 53) (width 0.2) (layer B.Cu) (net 15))
 (segment (start 159 53) (end 161 51) (width 0.2) (layer F.Cu) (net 15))
 (segment (start 143 53) (end 159 53) (width 0.2) (layer F.Cu) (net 15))
 (segment (start 101 63) (end 107.050002 63) (width 0.25) (layer F.Cu) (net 25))
 (segment (start 100 62) (end 101 63) (width 0.25) (layer F.Cu) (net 25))
 (segment (start 100 60) (end 100 62) (width 0.25) (layer F.Cu) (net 25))
 (segment (start 104 56) (end 100 60) (width 0.25) (layer F.Cu) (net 25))
 (segment (start 107.050002 63) (end 107.525001 62.525001) (width 0.25) (layer F.Cu) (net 25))
 (segment (start 115 56) (end 104 56) (width 0.25) (layer F.Cu) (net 25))
 (segment (start 141 60) (end 119 60) (width 0.25) (layer F.Cu) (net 25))
 (segment (start 119 60) (end 115 56) (width 0.25) (layer F.Cu) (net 25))
 (segment (start 119 58) (end 115 54) (width 0.25) (layer F.Cu) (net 24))
 (segment (start 114.63641 54) (end 104 54) (width 0.25) (layer F.Cu) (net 24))
 (segment (start 115 54) (end 114 54) (width 0.25) (layer F.Cu) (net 24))
 (segment (start 104 54) (end 98 60) (width 0.25) (layer F.Cu) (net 24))
 (via (at 98 64) (size 0.8) (drill 0.4) (layers F.Cu B.Cu) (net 24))
 (segment (start 98 60) (end 98 64) (width 0.25) (layer F.Cu) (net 24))
 (segment (start 107 64) (end 107.525001 64.525001) (width 0.25) (layer B.Cu) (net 24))
 (segment (start 98 64) (end 107 64) (width 0.25) (layer B.Cu) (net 24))
 (segment (start 125 56) (end 123 58) (width 0.25) (layer F.Cu) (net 24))
 (segment (start 119 58) (end 123 58) (width 0.25) (layer F.Cu) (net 24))
 (segment (start 125 56) (end 141 56) (width 0.25) (layer F.Cu) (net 24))
 (segment (start 142 55) (end 151 55) (width 0.25) (layer F.Cu) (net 24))
 (segment (start 141 56) (end 142 55) (width 0.25) (layer F.Cu) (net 24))
 (via (at 126 86) (size 0.8) (drill 0.4) (layers F.Cu B.Cu) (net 23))
 (segment (start 147 91) (end 132 91) (width 0.25) (layer F.Cu) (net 23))
 (segment (start 132 91) (end 127 86) (width 0.25) (layer F.Cu) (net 23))
 (segment (start 126 86) (end 127 86) (width 0.2) (layer F.Cu) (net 23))
 (segment (start 102 71) (end 106.474999 66.525001) (width 0.25) (layer B.Cu) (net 23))
 (segment (start 102 90) (end 102 71) (width 0.25) (layer B.Cu) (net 23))
 (segment (start 106.474999 66.525001) (end 107.525001 66.525001) (width 0.25) (layer B.Cu) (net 23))
 (segment (start 104 92) (end 102 90) (width 0.25) (layer B.Cu) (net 23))
 (segment (start 122 92) (end 104 92) (width 0.25) (layer B.Cu) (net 23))
 (segment (start 126 88) (end 122 92) (width 0.25) (layer B.Cu) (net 23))
 (segment (start 126 86) (end 126 88) (width 0.25) (layer B.Cu) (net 23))
 (via (at 125 85) (size 0.8) (drill 0.4) (layers F.Cu B.Cu) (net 22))
 (segment (start 141 88) (end 130 88) (width 0.25) (layer F.Cu) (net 22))
 (segment (start 130 88) (end 127 85) (width 0.25) (layer F.Cu) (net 22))
 (segment (start 125 85) (end 127 85) (width 0.2) (layer F.Cu) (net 22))
 (segment (start 105.474999 68.525001) (end 107.525001 68.525001) (width 0.25) (layer B.Cu) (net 22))
 (segment (start 103 71) (end 105.474999 68.525001) (width 0.25) (layer B.Cu) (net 22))
 (segment (start 103 90) (end 103 71) (width 0.25) (layer B.Cu) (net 22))
 (segment (start 104 91) (end 103 90) (width 0.25) (layer B.Cu) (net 22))
 (segment (start 121 91) (end 104 91) (width 0.25) (layer B.Cu) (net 22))
 (segment (start 125 87) (end 121 91) (width 0.25) (layer B.Cu) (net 22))
 (segment (start 125 85) (end 125 87) (width 0.25) (layer B.Cu) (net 22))
 (via (at 124 84) (size 0.8) (drill 0.4) (layers F.Cu B.Cu) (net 21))
 (segment (start 139 85) (end 138 84) (width 0.25) (layer F.Cu) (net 21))
 (segment (start 138 84) (end 124 84) (width 0.2) (layer F.Cu) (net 21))
 (segment (start 107 70) (end 107.525001 70.525001) (width 0.25) (layer B.Cu) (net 21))
 (segment (start 104 89) (end 104 72) (width 0.25) (layer B.Cu) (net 21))
 (segment (start 105 90) (end 104 89) (width 0.25) (layer B.Cu) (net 21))
 (segment (start 106 70) (end 107 70) (width 0.25) (layer B.Cu) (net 21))
 (segment (start 120 90) (end 105 90) (width 0.25) (layer B.Cu) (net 21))
 (segment (start 124 86) (end 120 90) (width 0.25) (layer B.Cu) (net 21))
 (segment (start 104 72) (end 106 70) (width 0.25) (layer B.Cu) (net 21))
 (segment (start 124 84) (end 124 86) (width 0.25) (layer B.Cu) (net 21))
 (segment (start 100.525001 80.525001) (end 107.525001 80.525001) (width 0.25) (layer F.Cu) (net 18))
 (segment (start 99 79) (end 100.525001 80.525001) (width 0.25) (layer F.Cu) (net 18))
 (segment (start 99 60) (end 99 79) (width 0.25) (layer F.Cu) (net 18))
 (segment (start 104 55) (end 99 60) (width 0.25) (layer F.Cu) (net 18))
 (segment (start 119 59) (end 115 55) (width 0.25) (layer F.Cu) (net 18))
 (segment (start 115 55) (end 104 55) (width 0.25) (layer F.Cu) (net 18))
 (segment (start 144 57) (end 126 57) (width 0.25) (layer F.Cu) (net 18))
 (segment (start 126 57) (end 124 59) (width 0.25) (layer F.Cu) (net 18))
 (segment (start 124 59) (end 119 59) (width 0.25) (layer F.Cu) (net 18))
 (segment (start 103 84) (end 104.474999 82.525001) (width 0.25) (layer F.Cu) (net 17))
 (segment (start 103 87) (end 103 84) (width 0.25) (layer F.Cu) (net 17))
 (segment (start 105 89) (end 103 87) (width 0.25) (layer F.Cu) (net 17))
 (segment (start 104.474999 82.525001) (end 107.525001 82.525001) (width 0.25) (layer F.Cu) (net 17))
 (segment (start 121 89) (end 105 89) (width 0.25) (layer F.Cu) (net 17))
 (segment (start 127 95) (end 121 89) (width 0.25) (layer F.Cu) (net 17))
 (segment (start 149 95) (end 127 95) (width 0.25) (layer F.Cu) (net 17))
 (segment (start 167.73 58) (end 168 57.73) (width 0.2) (layer F.Cu) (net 29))
 (segment (start 163 58) (end 167.73 58) (width 0.2) (layer F.Cu) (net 29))
 (segment (start 156.73 100.73) (end 157 101) (width 0.25) (layer F.Cu) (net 31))
 (segment (start 156.73 96) (end 156.73 100.73) (width 0.25) (layer F.Cu) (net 31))
 (segment (start 167.73 51) (end 168 50.73) (width 0.2) (layer F.Cu) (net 30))
 (segment (start 163 51) (end 167.73 51) (width 0.2) (layer F.Cu) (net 30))
 (segment (start 157 103) (end 146 103) (width 0.25) (layer F.Cu) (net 27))
 (segment (start 146 103) (end 144 101) (width 0.25) (layer F.Cu) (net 27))
 (via (at 144 101) (size 0.8) (drill 0.4) (layers F.Cu B.Cu) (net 27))
 (segment (start 117.474999 84.525001) (end 115.53 84.525001) (width 0.25) (layer B.Cu) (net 27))
 (segment (start 121 81) (end 117.474999 84.525001) (width 0.25) (layer B.Cu) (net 27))
 (segment (start 131 81) (end 121 81) (width 0.25) (layer B.Cu) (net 27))
 (segment (start 144 94) (end 131 81) (width 0.25) (layer B.Cu) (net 27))
 (segment (start 144 101) (end 144 94) (width 0.25) (layer B.Cu) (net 27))
 (segment (start 167.73 44) (end 168 43.73) (width 0.2) (layer F.Cu) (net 28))
 (segment (start 163 44) (end 167.73 44) (width 0.2) (layer F.Cu) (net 28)))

